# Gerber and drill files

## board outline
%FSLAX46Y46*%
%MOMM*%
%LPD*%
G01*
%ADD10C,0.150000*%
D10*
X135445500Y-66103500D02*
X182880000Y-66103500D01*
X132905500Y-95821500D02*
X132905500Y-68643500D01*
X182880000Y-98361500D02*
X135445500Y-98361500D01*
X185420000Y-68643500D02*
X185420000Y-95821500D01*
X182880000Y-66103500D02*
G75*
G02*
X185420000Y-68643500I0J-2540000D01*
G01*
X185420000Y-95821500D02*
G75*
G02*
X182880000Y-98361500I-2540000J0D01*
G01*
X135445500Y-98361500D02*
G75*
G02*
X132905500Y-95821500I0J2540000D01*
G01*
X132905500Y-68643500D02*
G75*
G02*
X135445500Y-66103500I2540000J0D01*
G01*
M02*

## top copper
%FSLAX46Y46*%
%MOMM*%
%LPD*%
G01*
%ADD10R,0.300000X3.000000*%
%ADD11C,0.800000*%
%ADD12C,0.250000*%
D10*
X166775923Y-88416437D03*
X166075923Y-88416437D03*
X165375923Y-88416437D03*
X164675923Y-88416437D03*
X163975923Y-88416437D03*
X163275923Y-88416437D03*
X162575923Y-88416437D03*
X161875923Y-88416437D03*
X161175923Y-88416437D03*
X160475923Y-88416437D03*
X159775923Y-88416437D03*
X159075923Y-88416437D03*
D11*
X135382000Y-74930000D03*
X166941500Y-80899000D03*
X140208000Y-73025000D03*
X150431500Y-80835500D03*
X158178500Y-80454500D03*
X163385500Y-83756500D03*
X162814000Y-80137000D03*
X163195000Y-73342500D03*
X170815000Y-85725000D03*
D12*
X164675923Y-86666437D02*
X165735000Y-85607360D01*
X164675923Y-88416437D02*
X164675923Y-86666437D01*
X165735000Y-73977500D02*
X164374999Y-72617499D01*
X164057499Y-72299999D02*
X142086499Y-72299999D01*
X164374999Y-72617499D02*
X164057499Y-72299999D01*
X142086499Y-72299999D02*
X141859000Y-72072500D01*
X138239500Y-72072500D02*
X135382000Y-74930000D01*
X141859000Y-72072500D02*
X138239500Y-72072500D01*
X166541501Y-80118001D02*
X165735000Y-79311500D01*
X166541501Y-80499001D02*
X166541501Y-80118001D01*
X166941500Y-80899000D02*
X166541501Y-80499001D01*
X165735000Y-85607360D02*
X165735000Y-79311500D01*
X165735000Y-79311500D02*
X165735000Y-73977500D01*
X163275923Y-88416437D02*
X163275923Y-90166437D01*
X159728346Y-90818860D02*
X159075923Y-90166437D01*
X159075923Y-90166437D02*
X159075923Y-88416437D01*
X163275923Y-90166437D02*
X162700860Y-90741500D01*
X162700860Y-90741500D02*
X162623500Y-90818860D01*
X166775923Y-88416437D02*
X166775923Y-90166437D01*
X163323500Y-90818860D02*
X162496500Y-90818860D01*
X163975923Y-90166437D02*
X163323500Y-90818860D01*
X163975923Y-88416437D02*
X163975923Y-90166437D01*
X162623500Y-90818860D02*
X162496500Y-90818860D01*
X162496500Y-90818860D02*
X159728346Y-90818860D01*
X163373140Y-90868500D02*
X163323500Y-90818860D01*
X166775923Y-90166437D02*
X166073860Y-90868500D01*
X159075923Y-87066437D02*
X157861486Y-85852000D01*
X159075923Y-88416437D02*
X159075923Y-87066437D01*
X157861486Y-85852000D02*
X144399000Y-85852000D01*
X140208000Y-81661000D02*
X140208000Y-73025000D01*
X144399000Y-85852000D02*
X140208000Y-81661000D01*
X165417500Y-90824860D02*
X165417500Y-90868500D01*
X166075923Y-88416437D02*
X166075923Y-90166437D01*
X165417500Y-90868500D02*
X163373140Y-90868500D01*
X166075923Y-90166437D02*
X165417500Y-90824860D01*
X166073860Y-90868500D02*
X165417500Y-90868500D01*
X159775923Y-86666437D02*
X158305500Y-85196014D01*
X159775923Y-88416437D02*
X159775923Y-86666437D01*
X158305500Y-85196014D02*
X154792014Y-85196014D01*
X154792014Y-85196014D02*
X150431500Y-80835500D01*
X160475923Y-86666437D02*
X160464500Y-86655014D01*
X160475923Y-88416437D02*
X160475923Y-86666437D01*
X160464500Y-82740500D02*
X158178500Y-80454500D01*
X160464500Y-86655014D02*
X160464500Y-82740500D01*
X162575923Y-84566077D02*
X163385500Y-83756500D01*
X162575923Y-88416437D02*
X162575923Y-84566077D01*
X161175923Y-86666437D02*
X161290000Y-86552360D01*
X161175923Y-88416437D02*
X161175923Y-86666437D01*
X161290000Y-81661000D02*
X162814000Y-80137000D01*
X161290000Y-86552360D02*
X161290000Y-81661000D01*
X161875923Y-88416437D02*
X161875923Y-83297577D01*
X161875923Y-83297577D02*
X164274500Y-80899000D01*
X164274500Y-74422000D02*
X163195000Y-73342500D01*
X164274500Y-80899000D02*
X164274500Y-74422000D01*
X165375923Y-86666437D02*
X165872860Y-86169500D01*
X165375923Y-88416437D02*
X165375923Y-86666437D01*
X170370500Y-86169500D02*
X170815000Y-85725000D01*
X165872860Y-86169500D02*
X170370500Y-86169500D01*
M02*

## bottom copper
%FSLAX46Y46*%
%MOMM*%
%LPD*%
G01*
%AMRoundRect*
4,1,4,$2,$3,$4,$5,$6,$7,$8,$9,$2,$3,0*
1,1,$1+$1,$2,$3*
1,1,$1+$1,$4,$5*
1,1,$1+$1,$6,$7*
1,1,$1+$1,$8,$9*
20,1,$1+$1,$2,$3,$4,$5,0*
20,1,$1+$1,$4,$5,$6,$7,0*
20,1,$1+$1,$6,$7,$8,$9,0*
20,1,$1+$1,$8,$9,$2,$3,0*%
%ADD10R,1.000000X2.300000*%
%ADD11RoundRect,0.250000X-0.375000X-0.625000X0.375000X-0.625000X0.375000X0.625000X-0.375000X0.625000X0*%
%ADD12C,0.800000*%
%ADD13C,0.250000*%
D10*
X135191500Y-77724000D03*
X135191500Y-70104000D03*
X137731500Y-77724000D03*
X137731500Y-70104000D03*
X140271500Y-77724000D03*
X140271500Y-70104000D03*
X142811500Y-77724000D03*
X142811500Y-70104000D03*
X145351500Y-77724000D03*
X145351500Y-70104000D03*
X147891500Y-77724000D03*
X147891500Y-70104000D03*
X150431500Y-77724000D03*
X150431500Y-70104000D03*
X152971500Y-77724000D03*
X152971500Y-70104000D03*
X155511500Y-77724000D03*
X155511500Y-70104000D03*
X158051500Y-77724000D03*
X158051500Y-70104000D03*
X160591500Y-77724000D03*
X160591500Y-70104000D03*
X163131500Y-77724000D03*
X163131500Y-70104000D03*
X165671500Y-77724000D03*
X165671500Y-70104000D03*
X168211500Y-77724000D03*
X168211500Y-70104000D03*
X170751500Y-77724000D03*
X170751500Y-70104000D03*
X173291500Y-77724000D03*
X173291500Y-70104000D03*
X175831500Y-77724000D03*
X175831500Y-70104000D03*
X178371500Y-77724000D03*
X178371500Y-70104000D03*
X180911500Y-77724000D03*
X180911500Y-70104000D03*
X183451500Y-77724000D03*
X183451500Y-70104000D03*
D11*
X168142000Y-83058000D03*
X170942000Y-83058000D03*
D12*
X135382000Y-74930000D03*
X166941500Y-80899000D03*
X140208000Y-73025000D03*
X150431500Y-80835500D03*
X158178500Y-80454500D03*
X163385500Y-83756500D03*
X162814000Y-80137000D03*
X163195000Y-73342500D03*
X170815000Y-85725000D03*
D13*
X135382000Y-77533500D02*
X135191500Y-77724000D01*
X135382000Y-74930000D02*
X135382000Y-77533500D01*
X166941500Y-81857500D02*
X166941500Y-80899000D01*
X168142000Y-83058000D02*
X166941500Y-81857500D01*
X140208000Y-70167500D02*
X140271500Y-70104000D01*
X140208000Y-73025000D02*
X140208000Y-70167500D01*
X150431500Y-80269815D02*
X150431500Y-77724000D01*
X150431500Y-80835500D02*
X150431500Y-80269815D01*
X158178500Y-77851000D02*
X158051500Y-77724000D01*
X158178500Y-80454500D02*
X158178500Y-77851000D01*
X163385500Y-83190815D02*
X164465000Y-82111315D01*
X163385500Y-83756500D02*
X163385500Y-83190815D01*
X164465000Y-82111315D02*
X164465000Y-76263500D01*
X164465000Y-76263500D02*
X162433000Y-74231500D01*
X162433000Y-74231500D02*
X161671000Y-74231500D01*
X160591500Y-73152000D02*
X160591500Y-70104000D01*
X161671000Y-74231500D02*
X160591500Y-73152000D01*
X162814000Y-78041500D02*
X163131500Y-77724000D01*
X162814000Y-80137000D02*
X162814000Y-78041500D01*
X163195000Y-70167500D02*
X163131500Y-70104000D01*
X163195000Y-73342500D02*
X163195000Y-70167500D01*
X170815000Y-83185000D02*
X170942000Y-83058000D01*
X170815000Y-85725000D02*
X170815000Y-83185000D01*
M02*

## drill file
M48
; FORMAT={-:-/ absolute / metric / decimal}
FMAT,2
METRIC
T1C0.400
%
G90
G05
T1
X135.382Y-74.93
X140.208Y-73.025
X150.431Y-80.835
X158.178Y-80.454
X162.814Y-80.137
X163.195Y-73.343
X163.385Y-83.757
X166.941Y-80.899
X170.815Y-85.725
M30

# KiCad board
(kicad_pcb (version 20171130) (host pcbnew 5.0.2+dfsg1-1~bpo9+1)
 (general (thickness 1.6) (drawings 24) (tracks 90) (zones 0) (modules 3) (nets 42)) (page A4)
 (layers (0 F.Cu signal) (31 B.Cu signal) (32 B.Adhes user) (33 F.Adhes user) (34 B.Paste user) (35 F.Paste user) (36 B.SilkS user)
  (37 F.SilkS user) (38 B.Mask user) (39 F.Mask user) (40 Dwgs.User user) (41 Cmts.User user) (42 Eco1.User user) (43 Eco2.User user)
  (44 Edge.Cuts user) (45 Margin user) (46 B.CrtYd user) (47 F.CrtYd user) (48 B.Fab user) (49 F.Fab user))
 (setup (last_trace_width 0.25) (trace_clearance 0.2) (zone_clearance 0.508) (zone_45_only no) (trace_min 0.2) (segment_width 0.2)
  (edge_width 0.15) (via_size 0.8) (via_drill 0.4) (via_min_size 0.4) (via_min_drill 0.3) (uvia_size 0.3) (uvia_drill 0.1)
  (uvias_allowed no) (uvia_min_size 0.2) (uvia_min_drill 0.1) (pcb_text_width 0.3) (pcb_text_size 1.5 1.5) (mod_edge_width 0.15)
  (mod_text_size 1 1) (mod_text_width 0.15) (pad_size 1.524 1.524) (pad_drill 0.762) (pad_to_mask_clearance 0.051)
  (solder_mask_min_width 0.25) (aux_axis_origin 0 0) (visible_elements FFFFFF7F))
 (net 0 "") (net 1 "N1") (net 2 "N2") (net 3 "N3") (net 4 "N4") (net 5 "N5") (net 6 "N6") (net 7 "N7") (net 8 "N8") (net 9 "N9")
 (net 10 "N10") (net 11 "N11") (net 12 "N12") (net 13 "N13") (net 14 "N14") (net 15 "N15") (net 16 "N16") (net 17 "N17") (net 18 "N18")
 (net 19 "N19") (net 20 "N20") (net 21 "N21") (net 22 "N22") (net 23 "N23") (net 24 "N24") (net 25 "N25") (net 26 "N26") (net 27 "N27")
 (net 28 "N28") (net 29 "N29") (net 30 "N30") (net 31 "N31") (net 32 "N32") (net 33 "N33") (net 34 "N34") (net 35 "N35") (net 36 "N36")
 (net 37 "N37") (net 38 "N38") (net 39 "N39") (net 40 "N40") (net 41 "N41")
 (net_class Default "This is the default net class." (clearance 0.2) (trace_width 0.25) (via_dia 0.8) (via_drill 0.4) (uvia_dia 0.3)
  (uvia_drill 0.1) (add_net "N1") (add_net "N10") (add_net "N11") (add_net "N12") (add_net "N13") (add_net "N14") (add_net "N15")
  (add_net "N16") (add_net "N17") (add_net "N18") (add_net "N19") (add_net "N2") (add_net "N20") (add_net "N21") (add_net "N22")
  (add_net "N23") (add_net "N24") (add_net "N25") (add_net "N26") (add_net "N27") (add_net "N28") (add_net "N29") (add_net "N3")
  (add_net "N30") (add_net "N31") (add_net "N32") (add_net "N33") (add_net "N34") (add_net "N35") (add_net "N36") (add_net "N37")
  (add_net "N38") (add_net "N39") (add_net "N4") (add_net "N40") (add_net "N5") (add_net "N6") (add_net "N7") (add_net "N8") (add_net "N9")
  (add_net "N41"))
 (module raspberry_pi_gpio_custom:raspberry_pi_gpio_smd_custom (layer B.Cu) (at 159.3215 73.914)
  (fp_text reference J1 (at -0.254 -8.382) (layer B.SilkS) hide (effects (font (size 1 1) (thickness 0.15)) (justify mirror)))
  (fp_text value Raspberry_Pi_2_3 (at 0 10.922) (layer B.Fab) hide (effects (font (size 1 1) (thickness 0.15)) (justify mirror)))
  (pad 1 smd rect (at -24.13 3.81) (size 1 2.3) (layers B.Cu B.Paste B.Mask) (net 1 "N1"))
  (pad 2 smd rect (at -24.13 -3.81) (size 1 2.3) (layers B.Cu B.Paste B.Mask) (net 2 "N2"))
  (pad 3 smd rect (at -21.59 3.81) (size 1 2.3) (layers B.Cu B.Paste B.Mask) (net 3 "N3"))
  (pad 4 smd rect (at -21.59 -3.81) (size 1 2.3) (layers B.Cu B.Paste B.Mask) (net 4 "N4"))
  (pad 5 smd rect (at -19.05 3.81) (size 1 2.3) (layers B.Cu B.Paste B.Mask) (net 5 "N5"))
  (pad 6 smd rect (at -19.05 -3.81) (size 1 2.3) (layers B.Cu B.Paste B.Mask) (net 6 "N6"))
  (pad 7 smd rect (at -16.51 3.81) (size 1 2.3) (layers B.Cu B.Paste B.Mask) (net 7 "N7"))
  (pad 8 smd rect (at -16.51 -3.81) (size 1 2.3) (layers B.Cu B.Paste B.Mask) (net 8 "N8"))
  (pad 9 smd rect (at -13.97 3.81) (size 1 2.3) (layers B.Cu B.Paste B.Mask) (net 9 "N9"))
  (pad 10 smd rect (at -13.97 -3.81) (size 1 2.3) (layers B.Cu B.Paste B.Mask) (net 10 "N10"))
  (pad 11 smd rect (at -11.43 3.81) (size 1 2.3) (layers B.Cu B.Paste B.Mask) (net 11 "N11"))
  (pad 12 smd rect (at -11.43 -3.81) (size 1 2.3) (layers B.Cu B.Paste B.Mask) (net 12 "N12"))
  (pad 13 smd rect (at -8.89 3.81) (size 1 2.3) (layers B.Cu B.Paste B.Mask) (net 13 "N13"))
  (pad 14 smd rect (at -8.89 -3.81) (size 1 2.3) (layers B.Cu B.Paste B.Mask) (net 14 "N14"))
  (pad 15 smd rect (at -6.35 3.81) (size 1 2.3) (layers B.Cu B.Paste B.Mask) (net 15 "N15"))
  (pad 16 smd rect (at -6.35 -3.81) (size 1 2.3) (layers B.Cu B.Paste B.Mask) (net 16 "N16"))
  (pad 17 smd rect (at -3.81 3.81) (size 1 2.3) (layers B.Cu B.Paste B.Mask) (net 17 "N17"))
  (pad 18 smd rect (at -3.81 -3.81) (size 1 2.3) (layers B.Cu B.Paste B.Mask) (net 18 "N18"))
  (pad 19 smd rect (at -1.27 3.81) (size 1 2.3) (layers B.Cu B.Paste B.Mask) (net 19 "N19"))
  (pad 20 smd rect (at -1.27 -3.81) (size 1 2.3) (layers B.Cu B.Paste B.Mask) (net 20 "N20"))
  (pad 21 smd rect (at 1.27 3.81) (size 1 2.3) (layers B.Cu B.Paste B.Mask) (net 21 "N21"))
  (pad 22 smd rect (at 1.27 -3.81) (size 1 2.3) (layers B.Cu B.Paste B.Mask) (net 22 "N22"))
  (pad 23 smd rect (at 3.81 3.81) (size 1 2.3) (layers B.Cu B.Paste B.Mask) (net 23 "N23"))
  (pad 24 smd rect (at 3.81 -3.81) (size 1 2.3) (layers B.Cu B.Paste B.Mask) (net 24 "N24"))
  (pad 25 smd rect (at 6.35 3.81) (size 1 2.3) (layers B.Cu B.Paste B.Mask) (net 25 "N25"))
  (pad 26 smd rect (at 6.35 -3.81) (size 1 2.3) (layers B.Cu B.Paste B.Mask) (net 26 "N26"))
  (pad 27 smd rect (at 8.89 3.81) (size 1 2.3) (layers B.Cu B.Paste B.Mask) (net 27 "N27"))
  (pad 28 smd rect (at 8.89 -3.81) (size 1 2.3) (layers B.Cu B.Paste B.Mask) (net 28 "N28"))
  (pad 29 smd rect (at 11.43 3.81) (size 1 2.3) (layers B.Cu B.Paste B.Mask) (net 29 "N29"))
  (pad 30 smd rect (at 11.43 -3.81) (size 1 2.3) (layers B.Cu B.Paste B.Mask) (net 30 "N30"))
  (pad 31 smd rect (at 13.97 3.81) (size 1 2.3) (layers B.Cu B.Paste B.Mask) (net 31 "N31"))
  (pad 32 smd rect (at 13.97 -3.81) (size 1 2.3) (layers B.Cu B.Paste B.Mask) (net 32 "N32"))
  (pad 33 smd rect (at 16.51 3.81) (size 1 2.3) (layers B.Cu B.Paste B.Mask) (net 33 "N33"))
  (pad 34 smd rect (at 16.51 -3.81) (size 1 2.3) (layers B.Cu B.Paste B.Mask) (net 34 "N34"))
  (pad 35 smd rect (at 19.05 3.81) (size 1 2.3) (layers B.Cu B.Paste B.Mask) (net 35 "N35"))
  (pad 36 smd rect (at 19.05 -3.81) (size 1 2.3) (layers B.Cu B.Paste B.Mask) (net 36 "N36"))
  (pad 37 smd rect (at 21.59 3.81) (size 1 2.3) (layers B.Cu B.Paste B.Mask) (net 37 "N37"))
  (pad 38 smd rect (at 21.59 -3.81) (size 1 2.3) (layers B.Cu B.Paste B.Mask) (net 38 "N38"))
  (pad 39 smd rect (at 24.13 3.81) (size 1 2.3) (layers B.Cu B.Paste B.Mask) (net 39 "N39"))
  (pad 40 smd rect (at 24.13 -3.81) (size 1 2.3) (layers B.Cu B.Paste B.Mask) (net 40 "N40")))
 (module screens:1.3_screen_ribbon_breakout (layer F.Cu) (at 162.941 89.916)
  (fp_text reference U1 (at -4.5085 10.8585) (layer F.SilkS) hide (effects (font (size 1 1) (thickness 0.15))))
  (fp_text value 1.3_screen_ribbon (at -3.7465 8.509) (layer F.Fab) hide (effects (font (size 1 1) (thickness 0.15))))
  (pad 1 smd rect (at 3.834923 -1.499563 180) (size 0.3 3) (layers F.Cu F.Paste F.Mask) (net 6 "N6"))
  (pad 2 smd rect (at 3.134923 -1.499563 180) (size 0.3 3) (layers F.Cu F.Paste F.Mask) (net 6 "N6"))
  (pad 3 smd rect (at 2.434923 -1.499563 180) (size 0.3 3) (layers F.Cu F.Paste F.Mask) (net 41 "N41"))
  (pad 4 smd rect (at 1.734923 -1.499563 180) (size 0.3 3) (layers F.Cu F.Paste F.Mask) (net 1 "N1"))
  (pad 5 smd rect (at 1.034923 -1.499563 180) (size 0.3 3) (layers F.Cu F.Paste F.Mask) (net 6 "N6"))
  (pad 6 smd rect (at 0.334923 -1.499563 180) (size 0.3 3) (layers F.Cu F.Paste F.Mask) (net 6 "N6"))
  (pad 7 smd rect (at -0.365077 -1.499563 180) (size 0.3 3) (layers F.Cu F.Paste F.Mask) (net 22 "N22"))
  (pad 8 smd rect (at -1.065077 -1.499563 180) (size 0.3 3) (layers F.Cu F.Paste F.Mask) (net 24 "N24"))
  (pad 9 smd rect (at -1.765077 -1.499563 180) (size 0.3 3) (layers F.Cu F.Paste F.Mask) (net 23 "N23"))
  (pad 10 smd rect (at -2.465077 -1.499563 180) (size 0.3 3) (layers F.Cu F.Paste F.Mask) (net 19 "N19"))
  (pad 11 smd rect (at -3.165077 -1.499563 180) (size 0.3 3) (layers F.Cu F.Paste F.Mask) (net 13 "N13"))
  (pad 12 smd rect (at -3.865077 -1.499563 180) (size 0.3 3) (layers F.Cu F.Paste F.Mask) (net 6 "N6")))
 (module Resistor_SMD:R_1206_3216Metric (layer B.Cu) (at 169.542 83.058)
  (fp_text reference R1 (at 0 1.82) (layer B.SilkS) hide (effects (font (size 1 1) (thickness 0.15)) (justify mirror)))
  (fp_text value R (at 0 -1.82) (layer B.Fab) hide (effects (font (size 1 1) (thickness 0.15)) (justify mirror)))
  (pad 1 smd roundrect (at -1.4 0) (size 1.25 1.75) (layers B.Cu B.Paste B.Mask) (roundrect_rratio 0.2) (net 1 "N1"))
  (pad 2 smd roundrect (at 1.4 0) (size 1.25 1.75) (layers B.Cu B.Paste B.Mask) (roundrect_rratio 0.2) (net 41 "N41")))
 (gr_line (start 135.4455 66.1035) (end 182.88 66.1035) (layer Edge.Cuts) (width 0.15))
 (gr_line (start 132.9055 95.8215) (end 132.9055 68.6435) (layer Edge.Cuts) (width 0.15))
 (gr_line (start 182.88 98.3615) (end 135.4455 98.3615) (layer Edge.Cuts) (width 0.15))
 (gr_line (start 185.42 68.6435) (end 185.42 95.8215) (layer Edge.Cuts) (width 0.15))
 (gr_arc (start 182.88 68.6435) (end 185.42 68.6435) (angle -90) (layer Edge.Cuts) (width 0.15))
 (gr_arc (start 182.88 95.8215) (end 182.88 98.3615) (angle -90) (layer Edge.Cuts) (width 0.15))
 (gr_arc (start 135.4455 95.8215) (end 132.9055 95.8215) (angle -90) (layer Edge.Cuts) (width 0.15))
 (gr_arc (start 135.4455 68.6435) (end 135.4455 66.1035) (angle -90) (layer Edge.Cuts) (width 0.15))
 (segment (start 164.675923 86.666437) (end 165.735 85.60736) (width 0.25) (layer F.Cu) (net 1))
 (segment (start 164.675923 88.416437) (end 164.675923 86.666437) (width 0.25) (layer F.Cu) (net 1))
 (segment (start 165.735 73.9775) (end 164.374999 72.617499) (width 0.25) (layer F.Cu) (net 1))
 (segment (start 164.057499 72.299999) (end 142.086499 72.299999) (width 0.25) (layer F.Cu) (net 1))
 (segment (start 164.374999 72.617499) (end 164.057499 72.299999) (width 0.25) (layer F.Cu) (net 1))
 (segment (start 142.086499 72.299999) (end 141.859 72.0725) (width 0.25) (layer F.Cu) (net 1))
 (via (at 135.382 74.93) (size 0.8) (drill 0.4) (layers F.Cu B.Cu) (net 1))
 (segment (start 138.2395 72.0725) (end 135.382 74.93) (width 0.25) (layer F.Cu) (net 1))
 (segment (start 141.859 72.0725) (end 138.2395 72.0725) (width 0.25) (layer F.Cu) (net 1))
 (segment (start 135.382 77.5335) (end 135.1915 77.724) (width 0.25) (layer B.Cu) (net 1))
 (segment (start 135.382 74.93) (end 135.382 77.5335) (width 0.25) (layer B.Cu) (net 1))
 (via (at 166.9415 80.899) (size 0.8) (drill 0.4) (layers F.Cu B.Cu) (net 1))
 (segment (start 166.9415 81.8575) (end 166.9415 80.899) (width 0.25) (layer B.Cu) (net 1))
 (segment (start 168.142 83.058) (end 166.9415 81.8575) (width 0.25) (layer B.Cu) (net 1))
 (segment (start 166.541501 80.118001) (end 165.735 79.3115) (width 0.25) (layer F.Cu) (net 1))
 (segment (start 166.541501 80.499001) (end 166.541501 80.118001) (width 0.25) (layer F.Cu) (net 1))
 (segment (start 166.9415 80.899) (end 166.541501 80.499001) (width 0.25) (layer F.Cu) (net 1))
 (segment (start 165.735 85.60736) (end 165.735 79.3115) (width 0.25) (layer F.Cu) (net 1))
 (segment (start 165.735 79.3115) (end 165.735 73.9775) (width 0.25) (layer F.Cu) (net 1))
 (segment (start 163.275923 88.416437) (end 163.275923 90.166437) (width 0.25) (layer F.Cu) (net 6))
 (segment (start 159.728346 90.81886) (end 159.075923 90.166437) (width 0.25) (layer F.Cu) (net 6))
 (segment (start 159.075923 90.166437) (end 159.075923 88.416437) (width 0.25) (layer F.Cu) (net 6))
 (segment (start 163.275923 90.166437) (end 162.70086 90.7415) (width 0.25) (layer F.Cu) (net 6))
 (segment (start 162.70086 90.7415) (end 162.6235 90.81886) (width 0.25) (layer F.Cu) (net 6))
 (segment (start 166.775923 88.416437) (end 166.775923 90.166437) (width 0.25) (layer F.Cu) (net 6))
 (segment (start 163.3235 90.81886) (end 162.4965 90.81886) (width 0.25) (layer F.Cu) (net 6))
 (segment (start 163.975923 90.166437) (end 163.3235 90.81886) (width 0.25) (layer F.Cu) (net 6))
 (segment (start 163.975923 88.416437) (end 163.975923 90.166437) (width 0.25) (layer F.Cu) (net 6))
 (segment (start 162.6235 90.81886) (end 162.4965 90.81886) (width 0.25) (layer F.Cu) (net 6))
 (segment (start 162.4965 90.81886) (end 159.728346 90.81886) (width 0.25) (layer F.Cu) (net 6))
 (segment (start 163.37314 90.8685) (end 163.3235 90.81886) (width 0.25) (layer F.Cu) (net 6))
 (segment (start 166.775923 90.166437) (end 166.07386 90.8685) (width 0.25) (layer F.Cu) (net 6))
 (segment (start 159.075923 87.066437) (end 157.861486 85.852) (width 0.25) (layer F.Cu) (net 6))
 (segment (start 159.075923 88.416437) (end 159.075923 87.066437) (width 0.25) (layer F.Cu) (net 6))
 (segment (start 157.861486 85.852) (end 144.399 85.852) (width 0.25) (layer F.Cu) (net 6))
 (via (at 140.208 73.025) (size 0.8) (drill 0.4) (layers F.Cu B.Cu) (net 6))
 (segment (start 140.208 81.661) (end 140.208 73.025) (width 0.25) (layer F.Cu) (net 6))
 (segment (start 144.399 85.852) (end 140.208 81.661) (width 0.25) (layer F.Cu) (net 6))
 (segment (start 140.208 70.1675) (end 140.2715 70.104) (width 0.25) (layer B.Cu) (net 6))
 (segment (start 140.208 73.025) (end 140.208 70.1675) (width 0.25) (layer B.Cu) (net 6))
 (segment (start 165.4175 90.82486) (end 165.4175 90.8685) (width 0.25) (layer F.Cu) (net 6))
 (segment (start 166.075923 88.416437) (end 166.075923 90.166437) (width 0.25) (layer F.Cu) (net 6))
 (segment (start 165.4175 90.8685) (end 163.37314 90.8685) (width 0.25) (layer F.Cu) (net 6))
 (segment (start 166.075923 90.166437) (end 165.4175 90.82486) (width 0.25) (layer F.Cu) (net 6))
 (segment (start 166.07386 90.8685) (end 165.4175 90.8685) (width 0.25) (layer F.Cu) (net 6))
 (segment (start 159.775923 86.666437) (end 158.3055 85.196014) (width 0.25) (layer F.Cu) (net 13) (status 1000000))
 (segment (start 159.775923 88.416437) (end 159.775923 86.666437) (width 0.25) (layer F.Cu) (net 13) (status 1000000))
 (segment (start 150.4315 80.269815) (end 150.4315 77.724) (width 0.25) (layer B.Cu) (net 13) (status 1000000))
 (segment (start 158.3055 85.196014) (end 154.792014 85.196014) (width 0.25) (layer F.Cu) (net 13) (status 1000000))
 (segment (start 154.792014 85.196014) (end 150.4315 80.8355) (width 0.25) (layer F.Cu) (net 13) (status 1000000))
 (via (at 150.4315 80.8355) (size 0.8) (drill 0.4) (layers F.Cu B.Cu) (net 13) (status 1000000))
 (segment (start 150.4315 80.8355) (end 150.4315 80.269815) (width 0.25) (layer B.Cu) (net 13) (status 1000000))
 (segment (start 160.475923 86.666437) (end 160.4645 86.655014) (width 0.25) (layer F.Cu) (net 19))
 (segment (start 160.475923 88.416437) (end 160.475923 86.666437) (width 0.25) (layer F.Cu) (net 19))
 (via (at 158.1785 80.4545) (size 0.8) (drill 0.4) (layers F.Cu B.Cu) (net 19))
 (segment (start 160.4645 82.7405) (end 158.1785 80.4545) (width 0.25) (layer F.Cu) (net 19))
 (segment (start 160.4645 86.655014) (end 160.4645 82.7405) (width 0.25) (layer F.Cu) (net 19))
 (segment (start 158.1785 77.851) (end 158.0515 77.724) (width 0.25) (layer B.Cu) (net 19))
 (segment (start 158.1785 80.4545) (end 158.1785 77.851) (width 0.25) (layer B.Cu) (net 19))
 (via (at 163.3855 83.7565) (size 0.8) (drill 0.4) (layers F.Cu B.Cu) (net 22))
 (segment (start 162.575923 84.566077) (end 163.3855 83.7565) (width 0.25) (layer F.Cu) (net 22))
 (segment (start 162.575923 88.416437) (end 162.575923 84.566077) (width 0.25) (layer F.Cu) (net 22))
 (segment (start 163.3855 83.190815) (end 164.465 82.111315) (width 0.25) (layer B.Cu) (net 22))
 (segment (start 163.3855 83.7565) (end 163.3855 83.190815) (width 0.25) (layer B.Cu) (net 22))
 (segment (start 164.465 82.111315) (end 164.465 76.2635) (width 0.25) (layer B.Cu) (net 22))
 (segment (start 164.465 76.2635) (end 162.433 74.2315) (width 0.25) (layer B.Cu) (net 22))
 (segment (start 162.433 74.2315) (end 161.671 74.2315) (width 0.25) (layer B.Cu) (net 22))
 (segment (start 160.5915 73.152) (end 160.5915 70.104) (width 0.25) (layer B.Cu) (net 22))
 (segment (start 161.671 74.2315) (end 160.5915 73.152) (width 0.25) (layer B.Cu) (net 22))
 (segment (start 161.175923 86.666437) (end 161.29 86.55236) (width 0.25) (layer F.Cu) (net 23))
 (segment (start 161.175923 88.416437) (end 161.175923 86.666437) (width 0.25) (layer F.Cu) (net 23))
 (segment (start 161.29 81.661) (end 162.814 80.137) (width 0.25) (layer F.Cu) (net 23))
 (via (at 162.814 80.137) (size 0.8) (drill 0.4) (layers F.Cu B.Cu) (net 23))
 (segment (start 161.29 86.55236) (end 161.29 81.661) (width 0.25) (layer F.Cu) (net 23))
 (segment (start 162.814 78.0415) (end 163.1315 77.724) (width 0.25) (layer B.Cu) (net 23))
 (segment (start 162.814 80.137) (end 162.814 78.0415) (width 0.25) (layer B.Cu) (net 23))
 (segment (start 161.875923 88.416437) (end 161.875923 83.297577) (width 0.25) (layer F.Cu) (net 24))
 (segment (start 161.875923 83.297577) (end 164.2745 80.899) (width 0.25) (layer F.Cu) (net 24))
 (via (at 163.195 73.3425) (size 0.8) (drill 0.4) (layers F.Cu B.Cu) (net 24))
 (segment (start 164.2745 74.422) (end 163.195 73.3425) (width 0.25) (layer F.Cu) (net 24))
 (segment (start 164.2745 80.899) (end 164.2745 74.422) (width 0.25) (layer F.Cu) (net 24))
 (segment (start 163.195 70.1675) (end 163.1315 70.104) (width 0.25) (layer B.Cu) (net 24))
 (segment (start 163.195 73.3425) (end 163.195 70.1675) (width 0.25) (layer B.Cu) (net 24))
 (segment (start 165.375923 86.666437) (end 165.87286 86.1695) (width 0.25) (layer F.Cu) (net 41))
 (segment (start 165.375923 88.416437) (end 165.375923 86.666437) (width 0.25) (layer F.Cu) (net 41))
 (via (at 170.815 85.725) (size 0.8) (drill 0.4) (layers F.Cu B.Cu) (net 41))
 (segment (start 170.3705 86.1695) (end 170.815 85.725) (width 0.25) (layer F.Cu) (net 41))
 (segment (start 165.87286 86.1695) (end 170.3705 86.1695) (width 0.25) (layer F.Cu) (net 41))
 (segment (start 170.815 83.185) (end 170.942 83.058) (width 0.25) (layer B.Cu) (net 41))
 (segment (start 170.815 85.725) (end 170.815 83.185) (width 0.25) (layer B.Cu) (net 41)))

